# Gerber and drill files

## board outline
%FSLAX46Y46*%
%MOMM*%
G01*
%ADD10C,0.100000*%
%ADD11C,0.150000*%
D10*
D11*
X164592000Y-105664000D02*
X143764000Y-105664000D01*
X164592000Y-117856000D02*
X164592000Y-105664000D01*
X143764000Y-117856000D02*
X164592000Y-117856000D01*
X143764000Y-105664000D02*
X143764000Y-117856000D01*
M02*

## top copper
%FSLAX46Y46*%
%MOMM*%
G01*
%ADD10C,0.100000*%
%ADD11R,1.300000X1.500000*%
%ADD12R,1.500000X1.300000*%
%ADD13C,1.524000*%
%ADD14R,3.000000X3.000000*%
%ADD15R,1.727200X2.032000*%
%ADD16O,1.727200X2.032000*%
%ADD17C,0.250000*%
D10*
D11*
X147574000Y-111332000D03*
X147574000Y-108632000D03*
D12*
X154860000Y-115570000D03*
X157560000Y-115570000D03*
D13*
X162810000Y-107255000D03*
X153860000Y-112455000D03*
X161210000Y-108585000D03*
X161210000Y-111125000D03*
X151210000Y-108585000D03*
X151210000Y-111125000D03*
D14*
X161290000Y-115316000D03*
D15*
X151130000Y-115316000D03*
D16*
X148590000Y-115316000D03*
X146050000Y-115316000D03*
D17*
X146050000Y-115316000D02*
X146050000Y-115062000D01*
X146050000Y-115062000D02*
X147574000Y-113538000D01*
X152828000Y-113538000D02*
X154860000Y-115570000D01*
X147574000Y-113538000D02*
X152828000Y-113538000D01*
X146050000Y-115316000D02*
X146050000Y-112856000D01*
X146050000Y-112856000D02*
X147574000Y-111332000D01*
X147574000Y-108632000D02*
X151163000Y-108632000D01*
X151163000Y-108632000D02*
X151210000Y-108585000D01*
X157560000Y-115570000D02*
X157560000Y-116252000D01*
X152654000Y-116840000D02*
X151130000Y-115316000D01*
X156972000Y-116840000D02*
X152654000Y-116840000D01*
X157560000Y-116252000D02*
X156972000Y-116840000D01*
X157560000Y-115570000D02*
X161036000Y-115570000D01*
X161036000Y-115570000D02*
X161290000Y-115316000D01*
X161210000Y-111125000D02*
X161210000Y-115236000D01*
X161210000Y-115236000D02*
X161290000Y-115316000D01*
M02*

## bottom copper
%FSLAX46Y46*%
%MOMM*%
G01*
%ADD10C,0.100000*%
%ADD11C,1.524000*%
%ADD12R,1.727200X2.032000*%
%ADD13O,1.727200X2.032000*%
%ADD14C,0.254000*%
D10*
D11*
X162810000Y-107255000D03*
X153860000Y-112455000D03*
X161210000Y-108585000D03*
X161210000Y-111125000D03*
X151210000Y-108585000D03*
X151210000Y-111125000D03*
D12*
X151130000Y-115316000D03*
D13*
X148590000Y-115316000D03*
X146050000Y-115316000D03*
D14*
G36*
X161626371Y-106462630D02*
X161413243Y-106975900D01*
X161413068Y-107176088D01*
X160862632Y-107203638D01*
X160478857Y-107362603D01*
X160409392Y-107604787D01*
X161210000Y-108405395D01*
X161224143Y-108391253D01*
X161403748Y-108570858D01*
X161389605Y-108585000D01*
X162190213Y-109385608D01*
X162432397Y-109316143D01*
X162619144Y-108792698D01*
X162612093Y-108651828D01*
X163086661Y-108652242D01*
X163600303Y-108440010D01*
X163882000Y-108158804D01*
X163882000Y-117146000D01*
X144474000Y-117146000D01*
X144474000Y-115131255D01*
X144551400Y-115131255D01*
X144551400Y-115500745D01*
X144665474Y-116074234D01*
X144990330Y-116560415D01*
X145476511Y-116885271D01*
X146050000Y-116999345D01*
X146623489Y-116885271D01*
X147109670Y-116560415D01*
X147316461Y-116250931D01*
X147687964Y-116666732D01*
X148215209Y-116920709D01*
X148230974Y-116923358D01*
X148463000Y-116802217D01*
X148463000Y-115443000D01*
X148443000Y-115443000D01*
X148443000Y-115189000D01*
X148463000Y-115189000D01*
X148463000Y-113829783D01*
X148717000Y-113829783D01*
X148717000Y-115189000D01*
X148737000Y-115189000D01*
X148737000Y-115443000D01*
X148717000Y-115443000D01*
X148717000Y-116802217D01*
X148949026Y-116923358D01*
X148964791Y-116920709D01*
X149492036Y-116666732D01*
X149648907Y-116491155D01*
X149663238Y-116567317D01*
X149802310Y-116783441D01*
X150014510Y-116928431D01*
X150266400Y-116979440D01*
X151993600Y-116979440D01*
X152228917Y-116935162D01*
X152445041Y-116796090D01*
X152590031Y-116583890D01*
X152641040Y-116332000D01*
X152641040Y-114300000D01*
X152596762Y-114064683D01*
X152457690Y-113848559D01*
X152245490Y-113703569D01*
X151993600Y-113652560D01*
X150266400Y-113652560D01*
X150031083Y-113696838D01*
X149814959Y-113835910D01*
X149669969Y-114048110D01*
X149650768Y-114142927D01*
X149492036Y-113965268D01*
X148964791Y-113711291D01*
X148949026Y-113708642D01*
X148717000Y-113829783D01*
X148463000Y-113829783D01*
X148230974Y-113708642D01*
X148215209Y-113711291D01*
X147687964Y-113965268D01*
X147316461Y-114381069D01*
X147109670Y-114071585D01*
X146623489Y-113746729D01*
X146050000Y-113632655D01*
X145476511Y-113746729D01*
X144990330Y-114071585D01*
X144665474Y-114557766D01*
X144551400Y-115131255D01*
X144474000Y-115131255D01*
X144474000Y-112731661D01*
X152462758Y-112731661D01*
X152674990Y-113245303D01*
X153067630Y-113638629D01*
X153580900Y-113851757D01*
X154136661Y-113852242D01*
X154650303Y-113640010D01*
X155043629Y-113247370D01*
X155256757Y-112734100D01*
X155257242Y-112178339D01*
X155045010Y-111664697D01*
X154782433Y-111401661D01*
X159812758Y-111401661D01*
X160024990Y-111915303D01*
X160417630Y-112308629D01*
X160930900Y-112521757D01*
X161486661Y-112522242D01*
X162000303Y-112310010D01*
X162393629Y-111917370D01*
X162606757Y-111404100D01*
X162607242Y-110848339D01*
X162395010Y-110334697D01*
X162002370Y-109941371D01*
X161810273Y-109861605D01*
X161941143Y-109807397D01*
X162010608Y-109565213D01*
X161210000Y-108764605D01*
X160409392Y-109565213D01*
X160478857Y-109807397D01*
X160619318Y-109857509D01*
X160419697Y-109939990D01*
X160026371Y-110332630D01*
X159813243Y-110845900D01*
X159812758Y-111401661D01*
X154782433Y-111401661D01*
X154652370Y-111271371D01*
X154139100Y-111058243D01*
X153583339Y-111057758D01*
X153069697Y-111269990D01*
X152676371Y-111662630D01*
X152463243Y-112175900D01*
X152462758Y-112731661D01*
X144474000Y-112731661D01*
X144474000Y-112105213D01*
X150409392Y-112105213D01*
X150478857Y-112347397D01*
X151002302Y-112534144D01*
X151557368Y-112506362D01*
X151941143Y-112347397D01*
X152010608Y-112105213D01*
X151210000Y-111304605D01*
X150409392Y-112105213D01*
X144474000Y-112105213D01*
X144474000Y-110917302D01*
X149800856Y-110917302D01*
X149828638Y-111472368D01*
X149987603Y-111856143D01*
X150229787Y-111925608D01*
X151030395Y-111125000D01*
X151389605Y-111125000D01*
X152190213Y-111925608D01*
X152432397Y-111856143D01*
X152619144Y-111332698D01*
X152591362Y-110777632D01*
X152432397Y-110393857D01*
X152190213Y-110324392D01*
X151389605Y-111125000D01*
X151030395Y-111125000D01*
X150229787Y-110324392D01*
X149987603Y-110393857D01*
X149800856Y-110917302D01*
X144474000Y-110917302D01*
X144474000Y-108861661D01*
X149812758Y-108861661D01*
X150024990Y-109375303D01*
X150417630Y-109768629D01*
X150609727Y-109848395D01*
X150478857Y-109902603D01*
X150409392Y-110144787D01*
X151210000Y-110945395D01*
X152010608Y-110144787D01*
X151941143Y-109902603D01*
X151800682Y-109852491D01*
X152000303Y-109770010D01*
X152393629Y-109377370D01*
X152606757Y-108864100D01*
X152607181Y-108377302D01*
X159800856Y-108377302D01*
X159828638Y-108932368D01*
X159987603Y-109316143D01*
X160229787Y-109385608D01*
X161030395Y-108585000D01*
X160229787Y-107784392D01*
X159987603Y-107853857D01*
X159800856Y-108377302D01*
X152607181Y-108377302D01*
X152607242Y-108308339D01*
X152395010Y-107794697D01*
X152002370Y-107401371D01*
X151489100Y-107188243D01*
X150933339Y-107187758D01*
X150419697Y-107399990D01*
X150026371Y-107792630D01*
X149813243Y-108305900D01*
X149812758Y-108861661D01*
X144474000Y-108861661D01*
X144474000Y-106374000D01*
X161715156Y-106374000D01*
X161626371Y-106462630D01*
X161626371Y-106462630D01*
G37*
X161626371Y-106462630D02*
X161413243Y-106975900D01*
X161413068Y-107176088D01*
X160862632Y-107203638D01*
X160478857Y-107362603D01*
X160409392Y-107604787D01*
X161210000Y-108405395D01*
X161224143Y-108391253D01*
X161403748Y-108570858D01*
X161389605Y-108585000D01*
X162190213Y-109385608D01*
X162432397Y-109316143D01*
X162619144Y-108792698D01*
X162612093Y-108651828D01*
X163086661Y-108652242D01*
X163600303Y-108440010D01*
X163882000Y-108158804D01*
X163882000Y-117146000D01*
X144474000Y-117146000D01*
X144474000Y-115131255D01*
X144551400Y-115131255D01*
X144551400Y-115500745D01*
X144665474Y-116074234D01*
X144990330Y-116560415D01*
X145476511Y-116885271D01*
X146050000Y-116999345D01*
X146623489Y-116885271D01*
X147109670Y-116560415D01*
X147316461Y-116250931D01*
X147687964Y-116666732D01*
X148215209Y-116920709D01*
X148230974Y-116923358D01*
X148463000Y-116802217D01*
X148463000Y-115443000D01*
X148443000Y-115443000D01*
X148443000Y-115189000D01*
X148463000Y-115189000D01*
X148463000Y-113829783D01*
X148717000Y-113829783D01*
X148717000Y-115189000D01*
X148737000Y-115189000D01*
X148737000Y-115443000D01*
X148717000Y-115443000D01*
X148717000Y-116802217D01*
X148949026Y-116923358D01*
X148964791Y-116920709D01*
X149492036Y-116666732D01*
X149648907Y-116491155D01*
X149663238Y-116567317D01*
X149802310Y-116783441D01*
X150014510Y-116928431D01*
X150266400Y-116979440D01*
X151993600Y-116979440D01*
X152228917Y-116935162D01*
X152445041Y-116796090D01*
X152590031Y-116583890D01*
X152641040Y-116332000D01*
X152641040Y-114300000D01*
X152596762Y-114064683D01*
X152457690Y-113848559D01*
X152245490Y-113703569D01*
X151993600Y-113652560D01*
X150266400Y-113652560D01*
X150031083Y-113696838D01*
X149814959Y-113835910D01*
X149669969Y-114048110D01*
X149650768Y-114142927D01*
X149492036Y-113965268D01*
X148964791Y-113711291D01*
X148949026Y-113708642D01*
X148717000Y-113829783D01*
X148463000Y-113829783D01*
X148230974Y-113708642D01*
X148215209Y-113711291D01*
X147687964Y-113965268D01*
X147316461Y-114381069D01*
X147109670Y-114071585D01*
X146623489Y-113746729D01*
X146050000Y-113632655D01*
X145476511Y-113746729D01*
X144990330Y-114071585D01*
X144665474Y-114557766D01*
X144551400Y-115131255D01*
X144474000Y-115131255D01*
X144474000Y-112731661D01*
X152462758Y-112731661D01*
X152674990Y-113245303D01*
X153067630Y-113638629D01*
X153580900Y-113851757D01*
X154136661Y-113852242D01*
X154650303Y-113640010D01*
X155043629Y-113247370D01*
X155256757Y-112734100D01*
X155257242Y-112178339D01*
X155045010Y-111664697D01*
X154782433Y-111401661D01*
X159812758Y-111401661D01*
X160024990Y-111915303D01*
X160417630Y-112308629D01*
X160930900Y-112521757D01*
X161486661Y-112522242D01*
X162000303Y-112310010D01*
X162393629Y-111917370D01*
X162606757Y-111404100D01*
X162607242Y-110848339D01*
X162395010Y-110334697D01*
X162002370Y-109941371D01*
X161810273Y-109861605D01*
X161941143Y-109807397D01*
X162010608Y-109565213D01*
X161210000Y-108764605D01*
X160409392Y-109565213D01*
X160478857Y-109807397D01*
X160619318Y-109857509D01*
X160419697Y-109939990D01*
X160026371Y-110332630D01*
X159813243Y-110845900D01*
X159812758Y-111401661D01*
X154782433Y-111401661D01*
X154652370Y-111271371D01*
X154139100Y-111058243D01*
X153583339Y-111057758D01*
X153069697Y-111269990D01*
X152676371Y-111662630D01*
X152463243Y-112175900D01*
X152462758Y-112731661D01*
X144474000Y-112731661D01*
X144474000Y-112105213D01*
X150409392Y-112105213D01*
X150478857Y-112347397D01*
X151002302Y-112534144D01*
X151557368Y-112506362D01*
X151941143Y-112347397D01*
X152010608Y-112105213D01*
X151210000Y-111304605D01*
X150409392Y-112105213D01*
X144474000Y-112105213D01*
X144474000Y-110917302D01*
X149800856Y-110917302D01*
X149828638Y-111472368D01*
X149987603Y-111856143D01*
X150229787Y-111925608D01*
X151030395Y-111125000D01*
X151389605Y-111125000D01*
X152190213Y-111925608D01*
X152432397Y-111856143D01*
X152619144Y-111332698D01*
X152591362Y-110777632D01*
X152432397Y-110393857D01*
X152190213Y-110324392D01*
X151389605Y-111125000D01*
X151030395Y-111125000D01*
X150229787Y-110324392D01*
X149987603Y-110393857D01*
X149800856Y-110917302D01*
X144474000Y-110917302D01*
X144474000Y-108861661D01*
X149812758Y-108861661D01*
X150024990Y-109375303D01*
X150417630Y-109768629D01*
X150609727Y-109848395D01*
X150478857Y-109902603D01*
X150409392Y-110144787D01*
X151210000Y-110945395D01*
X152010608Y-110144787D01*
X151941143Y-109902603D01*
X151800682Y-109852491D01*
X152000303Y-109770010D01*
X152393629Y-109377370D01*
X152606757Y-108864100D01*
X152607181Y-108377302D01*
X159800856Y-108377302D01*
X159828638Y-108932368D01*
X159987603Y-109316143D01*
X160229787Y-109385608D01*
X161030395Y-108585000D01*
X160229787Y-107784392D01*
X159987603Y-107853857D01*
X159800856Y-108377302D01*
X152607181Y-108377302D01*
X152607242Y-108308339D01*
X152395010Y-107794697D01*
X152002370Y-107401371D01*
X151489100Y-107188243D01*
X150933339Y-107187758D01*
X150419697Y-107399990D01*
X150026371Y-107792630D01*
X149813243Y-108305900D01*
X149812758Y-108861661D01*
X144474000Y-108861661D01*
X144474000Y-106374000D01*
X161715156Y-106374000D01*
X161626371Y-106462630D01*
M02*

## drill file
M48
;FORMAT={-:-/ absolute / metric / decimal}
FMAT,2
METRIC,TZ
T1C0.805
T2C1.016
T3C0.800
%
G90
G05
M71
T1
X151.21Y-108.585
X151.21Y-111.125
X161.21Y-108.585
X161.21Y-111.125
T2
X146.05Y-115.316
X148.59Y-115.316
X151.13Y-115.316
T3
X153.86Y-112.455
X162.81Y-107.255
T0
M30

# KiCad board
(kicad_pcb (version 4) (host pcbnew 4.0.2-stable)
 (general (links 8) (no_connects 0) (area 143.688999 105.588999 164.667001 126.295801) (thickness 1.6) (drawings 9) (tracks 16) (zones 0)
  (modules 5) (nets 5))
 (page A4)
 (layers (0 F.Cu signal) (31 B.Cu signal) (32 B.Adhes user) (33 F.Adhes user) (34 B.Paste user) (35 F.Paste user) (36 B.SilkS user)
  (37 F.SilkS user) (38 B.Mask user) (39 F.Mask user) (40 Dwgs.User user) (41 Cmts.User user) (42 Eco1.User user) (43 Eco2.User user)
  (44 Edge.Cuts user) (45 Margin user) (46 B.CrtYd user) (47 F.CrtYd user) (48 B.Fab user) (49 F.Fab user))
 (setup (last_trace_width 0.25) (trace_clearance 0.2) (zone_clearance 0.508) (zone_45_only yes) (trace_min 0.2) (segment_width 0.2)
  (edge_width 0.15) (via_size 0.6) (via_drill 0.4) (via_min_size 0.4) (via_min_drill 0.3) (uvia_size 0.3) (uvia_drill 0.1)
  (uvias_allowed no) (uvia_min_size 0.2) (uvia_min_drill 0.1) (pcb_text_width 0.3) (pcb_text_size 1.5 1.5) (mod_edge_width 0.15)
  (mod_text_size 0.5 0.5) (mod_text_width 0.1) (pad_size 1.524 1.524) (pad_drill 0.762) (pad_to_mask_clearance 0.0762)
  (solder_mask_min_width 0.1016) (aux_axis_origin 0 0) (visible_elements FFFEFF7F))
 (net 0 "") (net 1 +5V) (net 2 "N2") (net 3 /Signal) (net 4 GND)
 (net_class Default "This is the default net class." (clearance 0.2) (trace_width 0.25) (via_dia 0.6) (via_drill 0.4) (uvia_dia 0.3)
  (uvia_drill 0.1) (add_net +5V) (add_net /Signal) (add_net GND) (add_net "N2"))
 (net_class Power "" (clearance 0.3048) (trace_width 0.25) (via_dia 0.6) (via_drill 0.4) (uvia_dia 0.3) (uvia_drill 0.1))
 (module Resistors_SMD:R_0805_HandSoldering (layer F.Cu) (at 147.574 109.982 90)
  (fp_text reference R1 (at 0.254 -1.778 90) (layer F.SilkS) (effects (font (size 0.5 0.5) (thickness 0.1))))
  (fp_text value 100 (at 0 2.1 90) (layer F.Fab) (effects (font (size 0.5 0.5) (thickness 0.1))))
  (pad 1 smd rect (at -1.35 0 90) (size 1.5 1.3) (layers F.Cu F.Paste F.Mask) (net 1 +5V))
  (pad 2 smd rect (at 1.35 0 90) (size 1.5 1.3) (layers F.Cu F.Paste F.Mask) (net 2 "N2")))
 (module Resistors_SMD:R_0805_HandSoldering (layer F.Cu) (at 156.21 115.57)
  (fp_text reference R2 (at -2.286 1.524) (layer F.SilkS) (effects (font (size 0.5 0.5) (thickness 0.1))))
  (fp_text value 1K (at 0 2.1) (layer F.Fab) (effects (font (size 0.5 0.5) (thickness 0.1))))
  (pad 1 smd rect (at -1.35 0) (size 1.5 1.3) (layers F.Cu F.Paste F.Mask) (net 1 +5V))
  (pad 2 smd rect (at 1.35 0) (size 1.5 1.3) (layers F.Cu F.Paste F.Mask) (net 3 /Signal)))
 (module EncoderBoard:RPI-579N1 (layer F.Cu) (at 156.21 109.855 180)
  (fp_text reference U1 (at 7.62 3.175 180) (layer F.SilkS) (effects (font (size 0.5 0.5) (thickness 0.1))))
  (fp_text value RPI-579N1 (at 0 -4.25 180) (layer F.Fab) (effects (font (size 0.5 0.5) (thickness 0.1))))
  (pad "" np_thru_hole circle (at -6.6 2.6 180) (size 1.524 1.524) (drill 0.8) (layers *.Cu *.Mask F.SilkS))
  (pad "" np_thru_hole circle (at 2.35 -2.6 180) (size 1.524 1.524) (drill 0.8) (layers *.Cu *.Mask F.SilkS))
  (pad 4 thru_hole circle (at -5 1.27 180) (size 1.524 1.524) (drill 0.805) (layers *.Cu *.Mask F.SilkS) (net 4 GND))
  (pad 3 thru_hole circle (at -5 -1.27 180) (size 1.524 1.524) (drill 0.805) (layers *.Cu *.Mask F.SilkS) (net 3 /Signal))
  (pad 1 thru_hole circle (at 5 1.27 180) (size 1.524 1.524) (drill 0.805) (layers *.Cu *.Mask F.SilkS) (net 2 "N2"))
  (pad 2 thru_hole circle (at 5 -1.27 180) (size 1.524 1.524) (drill 0.805) (layers *.Cu *.Mask F.SilkS) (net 4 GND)))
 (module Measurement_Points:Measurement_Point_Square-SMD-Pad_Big (layer F.Cu) (at 161.29 115.316)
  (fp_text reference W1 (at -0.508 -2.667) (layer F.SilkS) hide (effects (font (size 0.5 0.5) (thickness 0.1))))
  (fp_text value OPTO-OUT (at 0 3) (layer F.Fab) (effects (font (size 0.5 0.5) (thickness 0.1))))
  (pad 1 smd rect (at 0 0) (size 3 3) (layers F.Cu F.Mask) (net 3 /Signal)))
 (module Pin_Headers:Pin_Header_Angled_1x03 (layer F.Cu) (at 151.13 115.316 270)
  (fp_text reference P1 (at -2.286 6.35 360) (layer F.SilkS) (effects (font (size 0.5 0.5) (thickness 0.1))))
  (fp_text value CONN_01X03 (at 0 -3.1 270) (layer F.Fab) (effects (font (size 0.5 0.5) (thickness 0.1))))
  (pad 1 thru_hole rect (at 0 0 270) (size 2.032 1.7272) (drill 1.016) (layers *.Cu *.Mask F.SilkS) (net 3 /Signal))
  (pad 2 thru_hole oval (at 0 2.54 270) (size 2.032 1.7272) (drill 1.016) (layers *.Cu *.Mask F.SilkS) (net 4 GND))
  (pad 3 thru_hole oval (at 0 5.08 270) (size 2.032 1.7272) (drill 1.016) (layers *.Cu *.Mask F.SilkS) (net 1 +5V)))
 (gr_line (start 164.592 105.664) (end 143.764 105.664) (angle 90) (layer Edge.Cuts) (width 0.15))
 (gr_line (start 164.592 117.856) (end 164.592 105.664) (angle 90) (layer Edge.Cuts) (width 0.15))
 (gr_line (start 143.764 117.856) (end 164.592 117.856) (angle 90) (layer Edge.Cuts) (width 0.15))
 (gr_line (start 143.764 105.664) (end 143.764 117.856) (angle 90) (layer Edge.Cuts) (width 0.15))
 (segment (start 146.05 115.316) (end 146.05 115.062) (width 0.25) (layer F.Cu) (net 1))
 (segment (start 146.05 115.062) (end 147.574 113.538) (width 0.25) (layer F.Cu) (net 1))
 (segment (start 152.828 113.538) (end 154.86 115.57) (width 0.25) (layer F.Cu) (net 1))
 (segment (start 147.574 113.538) (end 152.828 113.538) (width 0.25) (layer F.Cu) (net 1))
 (segment (start 146.05 115.316) (end 146.05 112.856) (width 0.25) (layer F.Cu) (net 1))
 (segment (start 146.05 112.856) (end 147.574 111.332) (width 0.25) (layer F.Cu) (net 1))
 (segment (start 147.574 108.632) (end 151.163 108.632) (width 0.25) (layer F.Cu) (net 2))
 (segment (start 151.163 108.632) (end 151.21 108.585) (width 0.25) (layer F.Cu) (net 2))
 (segment (start 157.56 115.57) (end 157.56 116.252) (width 0.25) (layer F.Cu) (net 3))
 (segment (start 152.654 116.84) (end 151.13 115.316) (width 0.25) (layer F.Cu) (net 3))
 (segment (start 156.972 116.84) (end 152.654 116.84) (width 0.25) (layer F.Cu) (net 3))
 (segment (start 157.56 116.252) (end 156.972 116.84) (width 0.25) (layer F.Cu) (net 3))
 (segment (start 157.56 115.57) (end 161.036 115.57) (width 0.25) (layer F.Cu) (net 3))
 (segment (start 161.036 115.57) (end 161.29 115.316) (width 0.25) (layer F.Cu) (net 3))
 (segment (start 161.21 111.125) (end 161.21 115.236) (width 0.25) (layer F.Cu) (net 3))
 (segment (start 161.21 115.236) (end 161.29 115.316) (width 0.25) (layer F.Cu) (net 3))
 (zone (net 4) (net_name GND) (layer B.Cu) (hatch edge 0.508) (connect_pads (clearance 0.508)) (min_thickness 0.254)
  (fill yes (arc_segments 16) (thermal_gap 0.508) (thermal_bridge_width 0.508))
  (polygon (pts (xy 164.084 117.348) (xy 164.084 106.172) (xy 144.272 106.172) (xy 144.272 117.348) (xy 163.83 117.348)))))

